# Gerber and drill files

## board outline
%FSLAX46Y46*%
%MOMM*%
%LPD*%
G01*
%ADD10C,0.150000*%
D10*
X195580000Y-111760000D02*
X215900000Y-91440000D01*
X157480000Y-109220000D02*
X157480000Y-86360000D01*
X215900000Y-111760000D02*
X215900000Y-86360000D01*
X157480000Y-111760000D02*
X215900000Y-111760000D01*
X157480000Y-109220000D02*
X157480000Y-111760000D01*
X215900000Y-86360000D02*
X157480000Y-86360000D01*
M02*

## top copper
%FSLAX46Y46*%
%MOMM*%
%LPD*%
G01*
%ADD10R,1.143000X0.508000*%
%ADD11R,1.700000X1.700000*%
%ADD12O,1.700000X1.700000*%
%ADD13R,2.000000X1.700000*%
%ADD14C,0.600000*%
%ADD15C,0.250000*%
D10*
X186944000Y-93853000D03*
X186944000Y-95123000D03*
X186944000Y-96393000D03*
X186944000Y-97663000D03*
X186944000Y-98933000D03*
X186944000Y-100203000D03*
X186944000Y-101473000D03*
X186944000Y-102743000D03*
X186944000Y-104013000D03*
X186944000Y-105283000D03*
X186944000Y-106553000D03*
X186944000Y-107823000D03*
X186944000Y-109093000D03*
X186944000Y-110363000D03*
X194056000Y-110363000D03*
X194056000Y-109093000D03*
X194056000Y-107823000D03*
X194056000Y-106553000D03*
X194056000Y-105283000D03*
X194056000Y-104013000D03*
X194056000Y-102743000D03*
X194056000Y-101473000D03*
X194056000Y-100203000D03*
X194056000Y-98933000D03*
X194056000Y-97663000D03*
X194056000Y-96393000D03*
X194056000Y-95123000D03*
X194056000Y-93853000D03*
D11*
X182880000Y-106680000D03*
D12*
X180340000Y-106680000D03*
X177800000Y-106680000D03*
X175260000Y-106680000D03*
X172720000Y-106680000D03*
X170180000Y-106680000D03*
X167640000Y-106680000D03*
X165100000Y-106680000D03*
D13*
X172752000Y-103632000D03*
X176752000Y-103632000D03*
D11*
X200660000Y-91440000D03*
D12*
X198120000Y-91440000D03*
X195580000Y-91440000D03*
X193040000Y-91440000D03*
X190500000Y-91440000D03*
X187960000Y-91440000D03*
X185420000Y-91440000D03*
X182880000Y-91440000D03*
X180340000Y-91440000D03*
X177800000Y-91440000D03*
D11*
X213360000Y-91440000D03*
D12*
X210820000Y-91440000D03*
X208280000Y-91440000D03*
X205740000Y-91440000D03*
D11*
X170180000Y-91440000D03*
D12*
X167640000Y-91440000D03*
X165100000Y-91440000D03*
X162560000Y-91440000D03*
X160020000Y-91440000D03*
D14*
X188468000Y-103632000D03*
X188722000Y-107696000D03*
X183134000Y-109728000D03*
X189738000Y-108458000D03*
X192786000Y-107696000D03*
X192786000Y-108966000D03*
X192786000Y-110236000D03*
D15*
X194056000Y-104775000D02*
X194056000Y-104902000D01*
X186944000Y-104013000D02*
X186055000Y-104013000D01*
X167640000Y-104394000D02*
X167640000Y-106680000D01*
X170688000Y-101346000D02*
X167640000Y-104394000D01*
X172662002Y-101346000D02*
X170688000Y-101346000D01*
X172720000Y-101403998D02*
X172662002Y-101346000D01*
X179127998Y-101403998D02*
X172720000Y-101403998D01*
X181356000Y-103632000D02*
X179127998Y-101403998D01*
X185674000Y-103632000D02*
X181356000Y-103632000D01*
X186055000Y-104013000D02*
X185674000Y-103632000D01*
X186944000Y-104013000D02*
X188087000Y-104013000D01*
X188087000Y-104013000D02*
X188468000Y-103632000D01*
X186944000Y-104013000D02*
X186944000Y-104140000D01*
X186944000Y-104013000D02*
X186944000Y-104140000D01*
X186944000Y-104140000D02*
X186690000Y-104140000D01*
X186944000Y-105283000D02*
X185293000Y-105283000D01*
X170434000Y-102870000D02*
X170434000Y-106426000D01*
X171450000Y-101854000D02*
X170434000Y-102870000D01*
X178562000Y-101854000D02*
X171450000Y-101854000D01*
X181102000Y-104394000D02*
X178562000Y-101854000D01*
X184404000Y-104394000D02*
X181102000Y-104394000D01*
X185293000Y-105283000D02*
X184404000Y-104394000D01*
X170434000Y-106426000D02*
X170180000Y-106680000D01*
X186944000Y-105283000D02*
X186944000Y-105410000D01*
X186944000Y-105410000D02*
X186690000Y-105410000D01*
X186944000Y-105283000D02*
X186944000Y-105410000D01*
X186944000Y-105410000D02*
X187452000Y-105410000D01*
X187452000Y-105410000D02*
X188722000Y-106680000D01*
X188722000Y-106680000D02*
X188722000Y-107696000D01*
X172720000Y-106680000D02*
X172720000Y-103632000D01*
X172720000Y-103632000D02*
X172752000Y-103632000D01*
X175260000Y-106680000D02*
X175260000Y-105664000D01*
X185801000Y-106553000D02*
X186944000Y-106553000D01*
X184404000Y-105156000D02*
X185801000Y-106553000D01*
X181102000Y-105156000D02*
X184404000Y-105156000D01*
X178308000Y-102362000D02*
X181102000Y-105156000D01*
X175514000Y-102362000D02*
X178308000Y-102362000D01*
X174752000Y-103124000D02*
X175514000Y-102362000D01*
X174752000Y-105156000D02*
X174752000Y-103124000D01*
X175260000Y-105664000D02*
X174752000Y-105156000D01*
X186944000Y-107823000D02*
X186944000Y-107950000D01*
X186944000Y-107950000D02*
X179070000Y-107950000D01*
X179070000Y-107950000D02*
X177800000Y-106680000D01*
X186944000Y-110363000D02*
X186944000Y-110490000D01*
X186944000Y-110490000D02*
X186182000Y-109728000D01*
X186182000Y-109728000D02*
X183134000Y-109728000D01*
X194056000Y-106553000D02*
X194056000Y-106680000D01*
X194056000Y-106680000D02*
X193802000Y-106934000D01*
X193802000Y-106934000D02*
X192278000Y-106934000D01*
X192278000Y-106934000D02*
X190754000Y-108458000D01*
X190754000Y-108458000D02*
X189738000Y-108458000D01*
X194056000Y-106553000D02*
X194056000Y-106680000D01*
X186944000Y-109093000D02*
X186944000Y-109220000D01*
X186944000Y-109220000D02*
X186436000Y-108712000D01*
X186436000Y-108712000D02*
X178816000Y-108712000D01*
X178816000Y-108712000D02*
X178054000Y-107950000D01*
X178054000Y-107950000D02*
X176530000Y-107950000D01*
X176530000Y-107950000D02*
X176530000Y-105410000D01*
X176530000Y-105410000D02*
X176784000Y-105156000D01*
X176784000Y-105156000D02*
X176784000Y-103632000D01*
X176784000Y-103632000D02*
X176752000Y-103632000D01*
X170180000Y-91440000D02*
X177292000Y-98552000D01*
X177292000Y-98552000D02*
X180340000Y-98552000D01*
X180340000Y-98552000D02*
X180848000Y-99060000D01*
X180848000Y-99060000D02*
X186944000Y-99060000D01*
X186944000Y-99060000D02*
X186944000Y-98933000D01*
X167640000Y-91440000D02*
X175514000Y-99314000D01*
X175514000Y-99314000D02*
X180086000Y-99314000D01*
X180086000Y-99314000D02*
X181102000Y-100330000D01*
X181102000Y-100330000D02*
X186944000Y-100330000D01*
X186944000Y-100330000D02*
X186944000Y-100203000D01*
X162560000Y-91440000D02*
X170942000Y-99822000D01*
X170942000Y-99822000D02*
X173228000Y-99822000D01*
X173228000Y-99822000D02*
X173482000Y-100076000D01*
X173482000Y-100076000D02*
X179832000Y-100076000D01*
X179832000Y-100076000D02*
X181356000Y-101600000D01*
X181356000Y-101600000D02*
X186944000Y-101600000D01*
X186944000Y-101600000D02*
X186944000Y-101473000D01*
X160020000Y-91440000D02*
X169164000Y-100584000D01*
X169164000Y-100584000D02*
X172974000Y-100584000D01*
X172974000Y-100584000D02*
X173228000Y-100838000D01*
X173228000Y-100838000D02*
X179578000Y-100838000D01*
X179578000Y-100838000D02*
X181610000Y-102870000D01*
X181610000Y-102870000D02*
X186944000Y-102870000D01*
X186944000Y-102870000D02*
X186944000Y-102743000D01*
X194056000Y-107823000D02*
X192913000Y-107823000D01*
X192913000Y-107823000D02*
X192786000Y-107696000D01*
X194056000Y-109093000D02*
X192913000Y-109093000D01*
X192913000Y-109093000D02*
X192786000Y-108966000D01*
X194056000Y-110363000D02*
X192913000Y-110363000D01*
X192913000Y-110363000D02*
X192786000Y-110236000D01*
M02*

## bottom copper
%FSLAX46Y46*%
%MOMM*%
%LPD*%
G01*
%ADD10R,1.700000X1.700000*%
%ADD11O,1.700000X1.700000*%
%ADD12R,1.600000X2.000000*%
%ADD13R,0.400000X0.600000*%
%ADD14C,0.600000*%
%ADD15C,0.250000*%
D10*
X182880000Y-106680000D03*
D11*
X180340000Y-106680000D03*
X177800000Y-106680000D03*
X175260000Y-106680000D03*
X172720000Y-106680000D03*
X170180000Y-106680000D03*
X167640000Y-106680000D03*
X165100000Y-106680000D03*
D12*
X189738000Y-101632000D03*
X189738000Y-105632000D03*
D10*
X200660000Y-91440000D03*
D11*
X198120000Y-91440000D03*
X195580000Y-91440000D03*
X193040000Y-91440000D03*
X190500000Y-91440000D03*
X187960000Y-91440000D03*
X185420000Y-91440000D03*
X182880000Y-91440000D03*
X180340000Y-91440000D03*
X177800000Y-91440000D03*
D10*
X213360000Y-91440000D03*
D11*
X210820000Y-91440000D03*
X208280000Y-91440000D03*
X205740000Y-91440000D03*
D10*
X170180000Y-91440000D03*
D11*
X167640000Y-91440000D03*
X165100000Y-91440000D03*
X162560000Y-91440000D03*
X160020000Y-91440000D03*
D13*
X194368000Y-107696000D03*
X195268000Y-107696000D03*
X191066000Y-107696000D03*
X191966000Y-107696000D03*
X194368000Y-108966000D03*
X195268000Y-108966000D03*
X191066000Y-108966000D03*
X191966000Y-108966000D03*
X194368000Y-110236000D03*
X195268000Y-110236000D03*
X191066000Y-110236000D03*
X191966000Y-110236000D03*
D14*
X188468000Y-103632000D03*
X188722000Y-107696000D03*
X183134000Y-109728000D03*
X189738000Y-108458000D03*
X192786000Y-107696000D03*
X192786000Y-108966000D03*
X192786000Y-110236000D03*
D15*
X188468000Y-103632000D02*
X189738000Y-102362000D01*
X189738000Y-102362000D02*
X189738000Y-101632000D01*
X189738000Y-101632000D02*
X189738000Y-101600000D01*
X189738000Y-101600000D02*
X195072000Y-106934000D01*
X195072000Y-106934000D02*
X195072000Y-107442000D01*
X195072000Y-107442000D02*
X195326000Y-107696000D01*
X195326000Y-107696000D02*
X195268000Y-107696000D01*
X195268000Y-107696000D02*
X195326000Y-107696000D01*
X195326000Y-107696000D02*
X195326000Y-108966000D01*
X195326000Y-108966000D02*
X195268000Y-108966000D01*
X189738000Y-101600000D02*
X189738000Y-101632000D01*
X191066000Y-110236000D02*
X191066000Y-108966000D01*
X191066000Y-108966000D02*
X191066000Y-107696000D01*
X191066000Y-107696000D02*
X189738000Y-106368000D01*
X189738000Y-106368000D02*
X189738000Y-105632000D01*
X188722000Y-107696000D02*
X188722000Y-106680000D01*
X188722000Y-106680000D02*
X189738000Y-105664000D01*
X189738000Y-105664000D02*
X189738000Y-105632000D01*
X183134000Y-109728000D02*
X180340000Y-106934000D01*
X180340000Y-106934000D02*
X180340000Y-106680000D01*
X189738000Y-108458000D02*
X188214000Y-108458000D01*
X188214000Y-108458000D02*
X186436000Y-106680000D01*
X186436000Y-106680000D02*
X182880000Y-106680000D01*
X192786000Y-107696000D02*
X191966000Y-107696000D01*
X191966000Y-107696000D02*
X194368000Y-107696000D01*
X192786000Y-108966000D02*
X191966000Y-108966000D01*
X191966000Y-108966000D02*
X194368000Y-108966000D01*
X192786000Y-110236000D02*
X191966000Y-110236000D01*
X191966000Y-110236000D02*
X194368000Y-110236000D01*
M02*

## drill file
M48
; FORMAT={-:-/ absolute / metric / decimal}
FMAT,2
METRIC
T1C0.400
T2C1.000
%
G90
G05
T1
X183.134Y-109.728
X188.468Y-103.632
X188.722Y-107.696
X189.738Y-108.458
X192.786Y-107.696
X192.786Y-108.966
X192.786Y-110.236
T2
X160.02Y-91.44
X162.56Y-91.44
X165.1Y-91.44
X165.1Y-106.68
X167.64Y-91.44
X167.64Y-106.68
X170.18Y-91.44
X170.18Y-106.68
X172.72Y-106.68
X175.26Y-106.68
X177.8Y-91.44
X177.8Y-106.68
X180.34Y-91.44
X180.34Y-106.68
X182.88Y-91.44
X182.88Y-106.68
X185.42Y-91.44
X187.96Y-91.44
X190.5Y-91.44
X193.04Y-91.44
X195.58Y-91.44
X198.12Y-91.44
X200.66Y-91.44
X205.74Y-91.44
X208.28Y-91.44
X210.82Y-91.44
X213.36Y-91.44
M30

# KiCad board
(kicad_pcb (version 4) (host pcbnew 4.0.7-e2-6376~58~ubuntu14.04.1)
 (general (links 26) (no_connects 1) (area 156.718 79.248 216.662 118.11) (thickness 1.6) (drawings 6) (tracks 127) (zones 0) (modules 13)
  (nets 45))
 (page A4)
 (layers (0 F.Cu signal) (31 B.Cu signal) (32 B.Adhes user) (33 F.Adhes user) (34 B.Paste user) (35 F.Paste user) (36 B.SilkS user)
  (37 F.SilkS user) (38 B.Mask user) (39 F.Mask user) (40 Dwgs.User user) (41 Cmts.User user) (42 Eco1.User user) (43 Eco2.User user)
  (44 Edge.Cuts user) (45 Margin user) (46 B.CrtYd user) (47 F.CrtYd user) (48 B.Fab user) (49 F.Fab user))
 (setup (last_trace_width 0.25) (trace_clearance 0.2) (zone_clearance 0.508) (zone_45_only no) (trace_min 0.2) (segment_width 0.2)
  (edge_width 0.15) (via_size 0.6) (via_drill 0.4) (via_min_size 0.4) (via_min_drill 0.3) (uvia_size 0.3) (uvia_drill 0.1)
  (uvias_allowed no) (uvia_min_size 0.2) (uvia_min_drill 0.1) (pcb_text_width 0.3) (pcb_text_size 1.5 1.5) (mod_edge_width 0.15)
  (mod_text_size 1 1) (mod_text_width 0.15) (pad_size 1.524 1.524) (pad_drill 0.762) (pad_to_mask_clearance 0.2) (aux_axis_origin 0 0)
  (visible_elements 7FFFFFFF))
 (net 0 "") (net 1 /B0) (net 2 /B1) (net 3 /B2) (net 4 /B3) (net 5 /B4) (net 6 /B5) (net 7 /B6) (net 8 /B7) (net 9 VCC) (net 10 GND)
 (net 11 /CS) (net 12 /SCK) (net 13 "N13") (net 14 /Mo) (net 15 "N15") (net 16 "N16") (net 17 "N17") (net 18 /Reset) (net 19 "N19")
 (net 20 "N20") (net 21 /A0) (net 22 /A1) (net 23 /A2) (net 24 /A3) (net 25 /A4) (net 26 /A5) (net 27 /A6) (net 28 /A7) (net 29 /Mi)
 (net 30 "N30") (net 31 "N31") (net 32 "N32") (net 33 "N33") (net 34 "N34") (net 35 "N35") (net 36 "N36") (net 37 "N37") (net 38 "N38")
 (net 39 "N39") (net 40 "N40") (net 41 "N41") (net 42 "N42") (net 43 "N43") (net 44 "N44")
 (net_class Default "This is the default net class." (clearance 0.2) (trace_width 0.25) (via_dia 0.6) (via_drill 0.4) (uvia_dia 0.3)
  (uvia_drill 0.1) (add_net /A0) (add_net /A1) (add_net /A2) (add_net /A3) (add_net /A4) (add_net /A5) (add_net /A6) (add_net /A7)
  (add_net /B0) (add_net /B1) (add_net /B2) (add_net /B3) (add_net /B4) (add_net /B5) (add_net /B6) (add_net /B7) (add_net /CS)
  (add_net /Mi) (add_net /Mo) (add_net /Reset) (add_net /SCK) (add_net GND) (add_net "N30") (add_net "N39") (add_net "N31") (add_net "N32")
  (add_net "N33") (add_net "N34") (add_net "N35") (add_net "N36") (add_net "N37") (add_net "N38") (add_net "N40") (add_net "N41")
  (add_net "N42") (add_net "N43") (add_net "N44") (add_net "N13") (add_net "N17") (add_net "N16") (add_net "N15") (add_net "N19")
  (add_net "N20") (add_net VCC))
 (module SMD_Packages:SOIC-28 (layer F.Cu) (at 190.5 102.108 270)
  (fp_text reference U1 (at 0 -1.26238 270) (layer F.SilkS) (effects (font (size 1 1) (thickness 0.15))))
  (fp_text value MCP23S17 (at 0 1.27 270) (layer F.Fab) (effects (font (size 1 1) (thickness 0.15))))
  (pad 1 smd rect (at -8.255 3.556 270) (size 0.508 1.143) (layers F.Cu F.Paste F.Mask) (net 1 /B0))
  (pad 2 smd rect (at -6.985 3.556 270) (size 0.508 1.143) (layers F.Cu F.Paste F.Mask) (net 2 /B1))
  (pad 3 smd rect (at -5.715 3.556 270) (size 0.508 1.143) (layers F.Cu F.Paste F.Mask) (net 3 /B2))
  (pad 4 smd rect (at -4.445 3.556 270) (size 0.508 1.143) (layers F.Cu F.Paste F.Mask) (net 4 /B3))
  (pad 5 smd rect (at -3.175 3.556 270) (size 0.508 1.143) (layers F.Cu F.Paste F.Mask) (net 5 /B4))
  (pad 6 smd rect (at -1.905 3.556 270) (size 0.508 1.143) (layers F.Cu F.Paste F.Mask) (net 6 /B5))
  (pad 7 smd rect (at -0.635 3.556 270) (size 0.508 1.143) (layers F.Cu F.Paste F.Mask) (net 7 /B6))
  (pad 8 smd rect (at 0.635 3.556 270) (size 0.508 1.143) (layers F.Cu F.Paste F.Mask) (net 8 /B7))
  (pad 9 smd rect (at 1.905 3.556 270) (size 0.508 1.143) (layers F.Cu F.Paste F.Mask) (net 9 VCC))
  (pad 10 smd rect (at 3.175 3.556 270) (size 0.508 1.143) (layers F.Cu F.Paste F.Mask) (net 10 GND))
  (pad 11 smd rect (at 4.445 3.556 270) (size 0.508 1.143) (layers F.Cu F.Paste F.Mask) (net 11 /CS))
  (pad 12 smd rect (at 5.715 3.556 270) (size 0.508 1.143) (layers F.Cu F.Paste F.Mask) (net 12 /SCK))
  (pad 13 smd rect (at 6.985 3.556 270) (size 0.508 1.143) (layers F.Cu F.Paste F.Mask) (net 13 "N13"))
  (pad 14 smd rect (at 8.255 3.556 270) (size 0.508 1.143) (layers F.Cu F.Paste F.Mask) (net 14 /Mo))
  (pad 15 smd rect (at 8.255 -3.556 270) (size 0.508 1.143) (layers F.Cu F.Paste F.Mask) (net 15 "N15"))
  (pad 16 smd rect (at 6.985 -3.556 270) (size 0.508 1.143) (layers F.Cu F.Paste F.Mask) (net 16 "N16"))
  (pad 17 smd rect (at 5.715 -3.556 270) (size 0.508 1.143) (layers F.Cu F.Paste F.Mask) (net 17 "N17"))
  (pad 18 smd rect (at 4.445 -3.556 270) (size 0.508 1.143) (layers F.Cu F.Paste F.Mask) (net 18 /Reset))
  (pad 19 smd rect (at 3.175 -3.556 270) (size 0.508 1.143) (layers F.Cu F.Paste F.Mask) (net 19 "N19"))
  (pad 20 smd rect (at 1.905 -3.556 270) (size 0.508 1.143) (layers F.Cu F.Paste F.Mask) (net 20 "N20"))
  (pad 21 smd rect (at 0.635 -3.556 270) (size 0.508 1.143) (layers F.Cu F.Paste F.Mask) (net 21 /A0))
  (pad 22 smd rect (at -0.635 -3.556 270) (size 0.508 1.143) (layers F.Cu F.Paste F.Mask) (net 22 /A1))
  (pad 23 smd rect (at -1.905 -3.556 270) (size 0.508 1.143) (layers F.Cu F.Paste F.Mask) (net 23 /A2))
  (pad 24 smd rect (at -3.175 -3.556 270) (size 0.508 1.143) (layers F.Cu F.Paste F.Mask) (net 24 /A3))
  (pad 25 smd rect (at -4.445 -3.556 270) (size 0.508 1.143) (layers F.Cu F.Paste F.Mask) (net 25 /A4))
  (pad 26 smd rect (at -5.715 -3.556 270) (size 0.508 1.143) (layers F.Cu F.Paste F.Mask) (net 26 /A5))
  (pad 27 smd rect (at -6.985 -3.556 270) (size 0.508 1.143) (layers F.Cu F.Paste F.Mask) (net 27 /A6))
  (pad 28 smd rect (at -8.255 -3.556 270) (size 0.508 1.143) (layers F.Cu F.Paste F.Mask) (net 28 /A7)))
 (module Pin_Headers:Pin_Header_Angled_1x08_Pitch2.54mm (layer F.Cu) (at 182.88 106.68 270)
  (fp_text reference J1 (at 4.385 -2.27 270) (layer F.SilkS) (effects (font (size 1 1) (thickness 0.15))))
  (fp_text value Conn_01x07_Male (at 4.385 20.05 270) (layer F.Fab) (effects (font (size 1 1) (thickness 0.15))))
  (pad 1 thru_hole rect (at 0 0 270) (size 1.7 1.7) (drill 1) (layers *.Cu *.Mask) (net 18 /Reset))
  (pad 2 thru_hole oval (at 0 2.54 270) (size 1.7 1.7) (drill 1) (layers *.Cu *.Mask) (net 14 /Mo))
  (pad 3 thru_hole oval (at 0 5.08 270) (size 1.7 1.7) (drill 1) (layers *.Cu *.Mask) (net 12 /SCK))
  (pad 4 thru_hole oval (at 0 7.62 270) (size 1.7 1.7) (drill 1) (layers *.Cu *.Mask) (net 11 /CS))
  (pad 5 thru_hole oval (at 0 10.16 270) (size 1.7 1.7) (drill 1) (layers *.Cu *.Mask) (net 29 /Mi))
  (pad 6 thru_hole oval (at 0 12.7 270) (size 1.7 1.7) (drill 1) (layers *.Cu *.Mask) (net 10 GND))
  (pad 7 thru_hole oval (at 0 15.24 270) (size 1.7 1.7) (drill 1) (layers *.Cu *.Mask) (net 9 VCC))
  (pad 8 thru_hole oval (at 0 17.78 270) (size 1.7 1.7) (drill 1) (layers *.Cu *.Mask)))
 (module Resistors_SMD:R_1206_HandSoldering (layer F.Cu) (at 174.752 103.632)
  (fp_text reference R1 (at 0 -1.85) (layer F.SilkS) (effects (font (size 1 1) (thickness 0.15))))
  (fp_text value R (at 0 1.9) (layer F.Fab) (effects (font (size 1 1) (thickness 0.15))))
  (pad 1 smd rect (at -2 0) (size 2 1.7) (layers F.Cu F.Paste F.Mask) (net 29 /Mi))
  (pad 2 smd rect (at 2 0) (size 2 1.7) (layers F.Cu F.Paste F.Mask) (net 13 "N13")))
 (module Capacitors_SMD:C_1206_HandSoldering (layer B.Cu) (at 189.738 103.632 270)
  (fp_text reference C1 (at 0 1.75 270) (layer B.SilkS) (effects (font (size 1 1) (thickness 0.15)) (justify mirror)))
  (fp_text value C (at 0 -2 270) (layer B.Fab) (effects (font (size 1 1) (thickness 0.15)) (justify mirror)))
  (pad 1 smd rect (at -2 0 270) (size 2 1.6) (layers B.Cu B.Paste B.Mask) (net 9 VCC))
  (pad 2 smd rect (at 2 0 270) (size 2 1.6) (layers B.Cu B.Paste B.Mask) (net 10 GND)))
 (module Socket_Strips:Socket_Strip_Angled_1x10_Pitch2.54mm (layer F.Cu) (at 200.66 91.44 270)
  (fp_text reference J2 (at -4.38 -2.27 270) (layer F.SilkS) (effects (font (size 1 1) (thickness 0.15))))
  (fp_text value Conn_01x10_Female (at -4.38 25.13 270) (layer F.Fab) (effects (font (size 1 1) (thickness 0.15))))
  (pad 1 thru_hole rect (at 0 0 270) (size 1.7 1.7) (drill 1) (layers *.Cu *.Mask) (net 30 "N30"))
  (pad 2 thru_hole oval (at 0 2.54 270) (size 1.7 1.7) (drill 1) (layers *.Cu *.Mask) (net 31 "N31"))
  (pad 3 thru_hole oval (at 0 5.08 270) (size 1.7 1.7) (drill 1) (layers *.Cu *.Mask) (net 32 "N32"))
  (pad 4 thru_hole oval (at 0 7.62 270) (size 1.7 1.7) (drill 1) (layers *.Cu *.Mask) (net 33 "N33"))
  (pad 5 thru_hole oval (at 0 10.16 270) (size 1.7 1.7) (drill 1) (layers *.Cu *.Mask) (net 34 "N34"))
  (pad 6 thru_hole oval (at 0 12.7 270) (size 1.7 1.7) (drill 1) (layers *.Cu *.Mask) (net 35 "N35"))
  (pad 7 thru_hole oval (at 0 15.24 270) (size 1.7 1.7) (drill 1) (layers *.Cu *.Mask) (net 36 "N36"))
  (pad 8 thru_hole oval (at 0 17.78 270) (size 1.7 1.7) (drill 1) (layers *.Cu *.Mask) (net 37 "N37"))
  (pad 9 thru_hole oval (at 0 20.32 270) (size 1.7 1.7) (drill 1) (layers *.Cu *.Mask) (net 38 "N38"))
  (pad 10 thru_hole oval (at 0 22.86 270) (size 1.7 1.7) (drill 1) (layers *.Cu *.Mask) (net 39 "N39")))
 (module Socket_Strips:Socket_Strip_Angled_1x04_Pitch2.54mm (layer F.Cu) (at 213.36 91.44 270)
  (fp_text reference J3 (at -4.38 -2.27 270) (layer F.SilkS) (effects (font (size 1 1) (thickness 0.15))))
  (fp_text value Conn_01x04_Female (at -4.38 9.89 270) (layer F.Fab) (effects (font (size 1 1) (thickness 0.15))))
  (pad 1 thru_hole rect (at 0 0 270) (size 1.7 1.7) (drill 1) (layers *.Cu *.Mask) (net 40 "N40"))
  (pad 2 thru_hole oval (at 0 2.54 270) (size 1.7 1.7) (drill 1) (layers *.Cu *.Mask) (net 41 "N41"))
  (pad 3 thru_hole oval (at 0 5.08 270) (size 1.7 1.7) (drill 1) (layers *.Cu *.Mask) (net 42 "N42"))
  (pad 4 thru_hole oval (at 0 7.62 270) (size 1.7 1.7) (drill 1) (layers *.Cu *.Mask) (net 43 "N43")))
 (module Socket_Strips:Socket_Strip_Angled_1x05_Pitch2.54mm (layer F.Cu) (at 170.18 91.44 270)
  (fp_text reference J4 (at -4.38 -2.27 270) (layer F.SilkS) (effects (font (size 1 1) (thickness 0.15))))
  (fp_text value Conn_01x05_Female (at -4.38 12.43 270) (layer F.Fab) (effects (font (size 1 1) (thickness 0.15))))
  (pad 1 thru_hole rect (at 0 0 270) (size 1.7 1.7) (drill 1) (layers *.Cu *.Mask) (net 5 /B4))
  (pad 2 thru_hole oval (at 0 2.54 270) (size 1.7 1.7) (drill 1) (layers *.Cu *.Mask) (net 6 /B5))
  (pad 3 thru_hole oval (at 0 5.08 270) (size 1.7 1.7) (drill 1) (layers *.Cu *.Mask) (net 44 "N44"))
  (pad 4 thru_hole oval (at 0 7.62 270) (size 1.7 1.7) (drill 1) (layers *.Cu *.Mask) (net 7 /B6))
  (pad 5 thru_hole oval (at 0 10.16 270) (size 1.7 1.7) (drill 1) (layers *.Cu *.Mask) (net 8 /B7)))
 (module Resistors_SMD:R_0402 (layer B.Cu) (at 194.818 107.696)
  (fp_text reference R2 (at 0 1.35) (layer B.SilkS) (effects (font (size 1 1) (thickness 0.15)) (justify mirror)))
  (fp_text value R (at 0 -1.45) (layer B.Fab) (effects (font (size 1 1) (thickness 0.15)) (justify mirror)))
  (pad 1 smd rect (at -0.45 0) (size 0.4 0.6) (layers B.Cu B.Paste B.Mask) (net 17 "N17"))
  (pad 2 smd rect (at 0.45 0) (size 0.4 0.6) (layers B.Cu B.Paste B.Mask) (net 9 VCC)))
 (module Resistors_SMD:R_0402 (layer B.Cu) (at 191.516 107.696)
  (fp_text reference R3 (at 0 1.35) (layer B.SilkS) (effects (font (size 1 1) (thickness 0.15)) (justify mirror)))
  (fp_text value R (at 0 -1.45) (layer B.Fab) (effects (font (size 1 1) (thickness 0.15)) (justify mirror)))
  (pad 1 smd rect (at -0.45 0) (size 0.4 0.6) (layers B.Cu B.Paste B.Mask) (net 10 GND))
  (pad 2 smd rect (at 0.45 0) (size 0.4 0.6) (layers B.Cu B.Paste B.Mask) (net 17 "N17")))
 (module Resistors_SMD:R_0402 (layer B.Cu) (at 194.818 108.966)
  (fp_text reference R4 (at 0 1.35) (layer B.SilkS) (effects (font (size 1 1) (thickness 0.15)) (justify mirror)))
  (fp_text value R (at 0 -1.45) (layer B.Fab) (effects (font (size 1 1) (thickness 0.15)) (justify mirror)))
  (pad 1 smd rect (at -0.45 0) (size 0.4 0.6) (layers B.Cu B.Paste B.Mask) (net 16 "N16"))
  (pad 2 smd rect (at 0.45 0) (size 0.4 0.6) (layers B.Cu B.Paste B.Mask) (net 9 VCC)))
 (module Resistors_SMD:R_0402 (layer B.Cu) (at 191.516 108.966)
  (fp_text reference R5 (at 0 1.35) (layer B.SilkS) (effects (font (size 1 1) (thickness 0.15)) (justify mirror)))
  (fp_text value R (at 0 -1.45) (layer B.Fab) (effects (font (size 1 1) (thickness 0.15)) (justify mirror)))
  (pad 1 smd rect (at -0.45 0) (size 0.4 0.6) (layers B.Cu B.Paste B.Mask) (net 10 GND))
  (pad 2 smd rect (at 0.45 0) (size 0.4 0.6) (layers B.Cu B.Paste B.Mask) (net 16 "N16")))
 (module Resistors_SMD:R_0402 (layer B.Cu) (at 194.818 110.236)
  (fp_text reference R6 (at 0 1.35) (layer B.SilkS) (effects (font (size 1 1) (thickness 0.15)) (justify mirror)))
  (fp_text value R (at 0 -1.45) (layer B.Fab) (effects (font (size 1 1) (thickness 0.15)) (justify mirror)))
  (pad 1 smd rect (at -0.45 0) (size 0.4 0.6) (layers B.Cu B.Paste B.Mask) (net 15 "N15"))
  (pad 2 smd rect (at 0.45 0) (size 0.4 0.6) (layers B.Cu B.Paste B.Mask) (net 9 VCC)))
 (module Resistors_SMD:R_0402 (layer B.Cu) (at 191.516 110.236)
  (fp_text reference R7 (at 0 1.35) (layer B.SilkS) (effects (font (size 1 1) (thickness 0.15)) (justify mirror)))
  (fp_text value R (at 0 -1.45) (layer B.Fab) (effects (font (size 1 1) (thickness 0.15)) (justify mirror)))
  (pad 1 smd rect (at -0.45 0) (size 0.4 0.6) (layers B.Cu B.Paste B.Mask) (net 10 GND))
  (pad 2 smd rect (at 0.45 0) (size 0.4 0.6) (layers B.Cu B.Paste B.Mask) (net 15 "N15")))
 (gr_line (start 195.58 111.76) (end 215.9 91.44) (angle 90) (layer Edge.Cuts) (width 0.15))
 (gr_line (start 157.48 109.22) (end 157.48 86.36) (angle 90) (layer Edge.Cuts) (width 0.15))
 (gr_line (start 215.9 111.76) (end 215.9 86.36) (angle 90) (layer Edge.Cuts) (width 0.15))
 (gr_line (start 157.48 111.76) (end 215.9 111.76) (angle 90) (layer Edge.Cuts) (width 0.15))
 (gr_line (start 157.48 109.22) (end 157.48 111.76) (angle 90) (layer Edge.Cuts) (width 0.15))
 (gr_line (start 215.9 86.36) (end 157.48 86.36) (angle 90) (layer Edge.Cuts) (width 0.15))
 (segment (start 194.056 104.775) (end 194.056 104.902) (width 0.25) (layer F.Cu) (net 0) (status 80000))
 (segment (start 186.944 104.013) (end 186.055 104.013) (width 0.25) (layer F.Cu) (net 9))
 (segment (start 167.64 104.394) (end 167.64 106.68) (width 0.25) (layer F.Cu) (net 9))
 (segment (start 170.688 101.346) (end 167.64 104.394) (width 0.25) (layer F.Cu) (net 9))
 (segment (start 172.662002 101.346) (end 170.688 101.346) (width 0.25) (layer F.Cu) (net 9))
 (segment (start 172.72 101.403998) (end 172.662002 101.346) (width 0.25) (layer F.Cu) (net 9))
 (segment (start 179.127998 101.403998) (end 172.72 101.403998) (width 0.25) (layer F.Cu) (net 9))
 (segment (start 181.356 103.632) (end 179.127998 101.403998) (width 0.25) (layer F.Cu) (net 9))
 (segment (start 185.674 103.632) (end 181.356 103.632) (width 0.25) (layer F.Cu) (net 9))
 (segment (start 186.055 104.013) (end 185.674 103.632) (width 0.25) (layer F.Cu) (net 9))
 (segment (start 186.944 104.013) (end 188.087 104.013) (width 0.25) (layer F.Cu) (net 9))
 (segment (start 188.468 103.632) (end 189.738 102.362) (width 0.25) (layer B.Cu) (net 9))
 (via (at 188.468 103.632) (size 0.6) (drill 0.4) (layers F.Cu B.Cu) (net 9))
 (segment (start 188.087 104.013) (end 188.468 103.632) (width 0.25) (layer F.Cu) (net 9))
 (segment (start 189.738 102.362) (end 189.738 101.632) (width 0.25) (layer B.Cu) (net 9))
 (segment (start 189.738 101.632) (end 189.738 101.6) (width 0.25) (layer B.Cu) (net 9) (status 80000))
 (segment (start 189.738 101.6) (end 195.072 106.934) (width 0.25) (layer B.Cu) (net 9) (status 80000))
 (segment (start 195.072 106.934) (end 195.072 107.442) (width 0.25) (layer B.Cu) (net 9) (status 80000))
 (segment (start 195.072 107.442) (end 195.326 107.696) (width 0.25) (layer B.Cu) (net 9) (status 80000))
 (segment (start 195.326 107.696) (end 195.268 107.696) (width 0.25) (layer B.Cu) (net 9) (status 80000))
 (segment (start 195.268 107.696) (end 195.326 107.696) (width 0.25) (layer B.Cu) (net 9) (status 80000))
 (segment (start 195.326 107.696) (end 195.326 108.966) (width 0.25) (layer B.Cu) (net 9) (status 80000))
 (segment (start 195.326 108.966) (end 195.268 108.966) (width 0.25) (layer B.Cu) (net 9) (status 80000))
 (segment (start 186.944 104.013) (end 186.944 104.14) (width 0.25) (layer F.Cu) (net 9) (status 80000))
 (segment (start 186.944 104.013) (end 186.944 104.14) (width 0.25) (layer F.Cu) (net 9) (status 80000))
 (segment (start 186.944 104.14) (end 186.69 104.14) (width 0.25) (layer F.Cu) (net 9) (status 80000))
 (segment (start 189.738 101.6) (end 189.738 101.632) (width 0.25) (layer B.Cu) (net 9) (status 80000))
 (segment (start 186.944 105.283) (end 185.293 105.283) (width 0.25) (layer F.Cu) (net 10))
 (segment (start 170.434 102.87) (end 170.434 106.426) (width 0.25) (layer F.Cu) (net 10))
 (segment (start 171.45 101.854) (end 170.434 102.87) (width 0.25) (layer F.Cu) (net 10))
 (segment (start 178.562 101.854) (end 171.45 101.854) (width 0.25) (layer F.Cu) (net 10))
 (segment (start 181.102 104.394) (end 178.562 101.854) (width 0.25) (layer F.Cu) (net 10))
 (segment (start 184.404 104.394) (end 181.102 104.394) (width 0.25) (layer F.Cu) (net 10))
 (segment (start 185.293 105.283) (end 184.404 104.394) (width 0.25) (layer F.Cu) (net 10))
 (segment (start 170.434 106.426) (end 170.18 106.68) (width 0.25) (layer F.Cu) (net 10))
 (segment (start 191.066 110.236) (end 191.066 108.966) (width 0.25) (layer B.Cu) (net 10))
 (segment (start 191.066 108.966) (end 191.066 107.696) (width 0.25) (layer B.Cu) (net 10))
 (segment (start 191.066 107.696) (end 189.738 106.368) (width 0.25) (layer B.Cu) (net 10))
 (segment (start 189.738 106.368) (end 189.738 105.632) (width 0.25) (layer B.Cu) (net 10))
 (segment (start 186.944 105.283) (end 186.944 105.41) (width 0.25) (layer F.Cu) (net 10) (status 80000))
 (segment (start 186.944 105.41) (end 186.69 105.41) (width 0.25) (layer F.Cu) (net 10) (status 80000))
 (segment (start 186.944 105.283) (end 186.944 105.41) (width 0.25) (layer F.Cu) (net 10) (status 80000))
 (segment (start 186.944 105.41) (end 187.452 105.41) (width 0.25) (layer F.Cu) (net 10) (status 80000))
 (segment (start 187.452 105.41) (end 188.722 106.68) (width 0.25) (layer F.Cu) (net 10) (status 80000))
 (segment (start 188.722 106.68) (end 188.722 107.696) (width 0.25) (layer F.Cu) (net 10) (status 80000))
 (via (at 188.722 107.696) (size 0.6) (layers F.Cu B.Cu) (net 10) (status 80000))
 (segment (start 188.722 107.696) (end 188.722 106.68) (width 0.25) (layer B.Cu) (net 10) (status 80000))
 (segment (start 188.722 106.68) (end 189.738 105.664) (width 0.25) (layer B.Cu) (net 10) (status 80000))
 (segment (start 189.738 105.664) (end 189.738 105.632) (width 0.25) (layer B.Cu) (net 10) (status 80000))
 (segment (start 172.72 106.68) (end 172.72 103.632) (width 0.25) (layer F.Cu) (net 29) (status 80000))
 (segment (start 172.72 103.632) (end 172.752 103.632) (width 0.25) (layer F.Cu) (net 29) (status 80000))
 (segment (start 175.26 106.68) (end 175.26 105.664) (width 0.25) (layer F.Cu) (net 11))
 (segment (start 185.801 106.553) (end 186.944 106.553) (width 0.25) (layer F.Cu) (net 11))
 (segment (start 184.404 105.156) (end 185.801 106.553) (width 0.25) (layer F.Cu) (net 11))
 (segment (start 181.102 105.156) (end 184.404 105.156) (width 0.25) (layer F.Cu) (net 11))
 (segment (start 178.308 102.362) (end 181.102 105.156) (width 0.25) (layer F.Cu) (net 11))
 (segment (start 175.514 102.362) (end 178.308 102.362) (width 0.25) (layer F.Cu) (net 11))
 (segment (start 174.752 103.124) (end 175.514 102.362) (width 0.25) (layer F.Cu) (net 11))
 (segment (start 174.752 105.156) (end 174.752 103.124) (width 0.25) (layer F.Cu) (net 11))
 (segment (start 175.26 105.664) (end 174.752 105.156) (width 0.25) (layer F.Cu) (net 11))
 (segment (start 186.944 107.823) (end 186.944 107.95) (width 0.25) (layer F.Cu) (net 12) (status 80000))
 (segment (start 186.944 107.95) (end 179.07 107.95) (width 0.25) (layer F.Cu) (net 12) (status 80000))
 (segment (start 179.07 107.95) (end 177.8 106.68) (width 0.25) (layer F.Cu) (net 12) (status 80000))
 (segment (start 186.944 110.363) (end 186.944 110.49) (width 0.25) (layer F.Cu) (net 14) (status 80000))
 (segment (start 186.944 110.49) (end 186.182 109.728) (width 0.25) (layer F.Cu) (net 14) (status 80000))
 (segment (start 186.182 109.728) (end 183.134 109.728) (width 0.25) (layer F.Cu) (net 14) (status 80000))
 (via (at 183.134 109.728) (size 0.6) (layers F.Cu B.Cu) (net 14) (status 80000))
 (segment (start 183.134 109.728) (end 180.34 106.934) (width 0.25) (layer B.Cu) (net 14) (status 80000))
 (segment (start 180.34 106.934) (end 180.34 106.68) (width 0.25) (layer B.Cu) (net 14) (status 80000))
 (segment (start 194.056 106.553) (end 194.056 106.68) (width 0.25) (layer F.Cu) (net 18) (status 80000))
 (segment (start 194.056 106.68) (end 193.802 106.934) (width 0.25) (layer F.Cu) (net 18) (status 80000))
 (segment (start 193.802 106.934) (end 192.278 106.934) (width 0.25) (layer F.Cu) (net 18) (status 80000))
 (segment (start 192.278 106.934) (end 190.754 108.458) (width 0.25) (layer F.Cu) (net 18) (status 80000))
 (segment (start 190.754 108.458) (end 189.738 108.458) (width 0.25) (layer F.Cu) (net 18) (status 80000))
 (via (at 189.738 108.458) (size 0.6) (layers F.Cu B.Cu) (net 18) (status 80000))
 (segment (start 189.738 108.458) (end 188.214 108.458) (width 0.25) (layer B.Cu) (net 18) (status 80000))
 (segment (start 188.214 108.458) (end 186.436 106.68) (width 0.25) (layer B.Cu) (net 18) (status 80000))
 (segment (start 186.436 106.68) (end 182.88 106.68) (width 0.25) (layer B.Cu) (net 18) (status 80000))
 (segment (start 194.056 106.553) (end 194.056 106.68) (width 0.25) (layer F.Cu) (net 18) (status 80000))
 (segment (start 186.944 109.093) (end 186.944 109.22) (width 0.25) (layer F.Cu) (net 13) (status 80000))
 (segment (start 186.944 109.22) (end 186.436 108.712) (width 0.25) (layer F.Cu) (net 13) (status 80000))
 (segment (start 186.436 108.712) (end 178.816 108.712) (width 0.25) (layer F.Cu) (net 13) (status 80000))
 (segment (start 178.816 108.712) (end 178.054 107.95) (width 0.25) (layer F.Cu) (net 13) (status 80000))
 (segment (start 178.054 107.95) (end 176.53 107.95) (width 0.25) (layer F.Cu) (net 13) (status 80000))
 (segment (start 176.53 107.95) (end 176.53 105.41) (width 0.25) (layer F.Cu) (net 13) (status 80000))
 (segment (start 176.53 105.41) (end 176.784 105.156) (width 0.25) (layer F.Cu) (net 13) (status 80000))
 (segment (start 176.784 105.156) (end 176.784 103.632) (width 0.25) (layer F.Cu) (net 13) (status 80000))
 (segment (start 176.784 103.632) (end 176.752 103.632) (width 0.25) (layer F.Cu) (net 13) (status 80000))
 (segment (start 170.18 91.44) (end 177.292 98.552) (width 0.25) (layer F.Cu) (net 5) (status 80000))
 (segment (start 177.292 98.552) (end 180.34 98.552) (width 0.25) (layer F.Cu) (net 5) (status 80000))
 (segment (start 180.34 98.552) (end 180.848 99.06) (width 0.25) (layer F.Cu) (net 5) (status 80000))
 (segment (start 180.848 99.06) (end 186.944 99.06) (width 0.25) (layer F.Cu) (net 5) (status 80000))
 (segment (start 186.944 99.06) (end 186.944 98.933) (width 0.25) (layer F.Cu) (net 5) (status 80000))
 (segment (start 167.64 91.44) (end 175.514 99.314) (width 0.25) (layer F.Cu) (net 6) (status 80000))
 (segment (start 175.514 99.314) (end 180.086 99.314) (width 0.25) (layer F.Cu) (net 6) (status 80000))
 (segment (start 180.086 99.314) (end 181.102 100.33) (width 0.25) (layer F.Cu) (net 6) (status 80000))
 (segment (start 181.102 100.33) (end 186.944 100.33) (width 0.25) (layer F.Cu) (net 6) (status 80000))
 (segment (start 186.944 100.33) (end 186.944 100.203) (width 0.25) (layer F.Cu) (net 6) (status 80000))
 (segment (start 162.56 91.44) (end 170.942 99.822) (width 0.25) (layer F.Cu) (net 7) (status 80000))
 (segment (start 170.942 99.822) (end 173.228 99.822) (width 0.25) (layer F.Cu) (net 7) (status 80000))
 (segment (start 173.228 99.822) (end 173.482 100.076) (width 0.25) (layer F.Cu) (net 7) (status 80000))
 (segment (start 173.482 100.076) (end 179.832 100.076) (width 0.25) (layer F.Cu) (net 7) (status 80000))
 (segment (start 179.832 100.076) (end 181.356 101.6) (width 0.25) (layer F.Cu) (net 7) (status 80000))
 (segment (start 181.356 101.6) (end 186.944 101.6) (width 0.25) (layer F.Cu) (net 7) (status 80000))
 (segment (start 186.944 101.6) (end 186.944 101.473) (width 0.25) (layer F.Cu) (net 7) (status 80000))
 (segment (start 160.02 91.44) (end 169.164 100.584) (width 0.25) (layer F.Cu) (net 8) (status 80000))
 (segment (start 169.164 100.584) (end 172.974 100.584) (width 0.25) (layer F.Cu) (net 8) (status 80000))
 (segment (start 172.974 100.584) (end 173.228 100.838) (width 0.25) (layer F.Cu) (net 8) (status 80000))
 (segment (start 173.228 100.838) (end 179.578 100.838) (width 0.25) (layer F.Cu) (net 8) (status 80000))
 (segment (start 179.578 100.838) (end 181.61 102.87) (width 0.25) (layer F.Cu) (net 8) (status 80000))
 (segment (start 181.61 102.87) (end 186.944 102.87) (width 0.25) (layer F.Cu) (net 8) (status 80000))
 (segment (start 186.944 102.87) (end 186.944 102.743) (width 0.25) (layer F.Cu) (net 8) (status 80000))
 (segment (start 194.056 107.823) (end 192.913 107.823) (width 0.25) (layer F.Cu) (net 17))
 (segment (start 192.786 107.696) (end 191.966 107.696) (width 0.25) (layer B.Cu) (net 17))
 (via (at 192.786 107.696) (size 0.6) (drill 0.4) (layers F.Cu B.Cu) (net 17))
 (segment (start 192.913 107.823) (end 192.786 107.696) (width 0.25) (layer F.Cu) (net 17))
 (segment (start 191.966 107.696) (end 194.368 107.696) (width 0.25) (layer B.Cu) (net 17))
 (segment (start 194.056 109.093) (end 192.913 109.093) (width 0.25) (layer F.Cu) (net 16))
 (segment (start 192.786 108.966) (end 191.966 108.966) (width 0.25) (layer B.Cu) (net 16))
 (via (at 192.786 108.966) (size 0.6) (drill 0.4) (layers F.Cu B.Cu) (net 16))
 (segment (start 192.913 109.093) (end 192.786 108.966) (width 0.25) (layer F.Cu) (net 16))
 (segment (start 191.966 108.966) (end 194.368 108.966) (width 0.25) (layer B.Cu) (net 16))
 (segment (start 194.056 110.363) (end 192.913 110.363) (width 0.25) (layer F.Cu) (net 15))
 (segment (start 192.786 110.236) (end 191.966 110.236) (width 0.25) (layer B.Cu) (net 15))
 (via (at 192.786 110.236) (size 0.6) (drill 0.4) (layers F.Cu B.Cu) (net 15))
 (segment (start 192.913 110.363) (end 192.786 110.236) (width 0.25) (layer F.Cu) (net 15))
 (segment (start 191.966 110.236) (end 194.368 110.236) (width 0.25) (layer B.Cu) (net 15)))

